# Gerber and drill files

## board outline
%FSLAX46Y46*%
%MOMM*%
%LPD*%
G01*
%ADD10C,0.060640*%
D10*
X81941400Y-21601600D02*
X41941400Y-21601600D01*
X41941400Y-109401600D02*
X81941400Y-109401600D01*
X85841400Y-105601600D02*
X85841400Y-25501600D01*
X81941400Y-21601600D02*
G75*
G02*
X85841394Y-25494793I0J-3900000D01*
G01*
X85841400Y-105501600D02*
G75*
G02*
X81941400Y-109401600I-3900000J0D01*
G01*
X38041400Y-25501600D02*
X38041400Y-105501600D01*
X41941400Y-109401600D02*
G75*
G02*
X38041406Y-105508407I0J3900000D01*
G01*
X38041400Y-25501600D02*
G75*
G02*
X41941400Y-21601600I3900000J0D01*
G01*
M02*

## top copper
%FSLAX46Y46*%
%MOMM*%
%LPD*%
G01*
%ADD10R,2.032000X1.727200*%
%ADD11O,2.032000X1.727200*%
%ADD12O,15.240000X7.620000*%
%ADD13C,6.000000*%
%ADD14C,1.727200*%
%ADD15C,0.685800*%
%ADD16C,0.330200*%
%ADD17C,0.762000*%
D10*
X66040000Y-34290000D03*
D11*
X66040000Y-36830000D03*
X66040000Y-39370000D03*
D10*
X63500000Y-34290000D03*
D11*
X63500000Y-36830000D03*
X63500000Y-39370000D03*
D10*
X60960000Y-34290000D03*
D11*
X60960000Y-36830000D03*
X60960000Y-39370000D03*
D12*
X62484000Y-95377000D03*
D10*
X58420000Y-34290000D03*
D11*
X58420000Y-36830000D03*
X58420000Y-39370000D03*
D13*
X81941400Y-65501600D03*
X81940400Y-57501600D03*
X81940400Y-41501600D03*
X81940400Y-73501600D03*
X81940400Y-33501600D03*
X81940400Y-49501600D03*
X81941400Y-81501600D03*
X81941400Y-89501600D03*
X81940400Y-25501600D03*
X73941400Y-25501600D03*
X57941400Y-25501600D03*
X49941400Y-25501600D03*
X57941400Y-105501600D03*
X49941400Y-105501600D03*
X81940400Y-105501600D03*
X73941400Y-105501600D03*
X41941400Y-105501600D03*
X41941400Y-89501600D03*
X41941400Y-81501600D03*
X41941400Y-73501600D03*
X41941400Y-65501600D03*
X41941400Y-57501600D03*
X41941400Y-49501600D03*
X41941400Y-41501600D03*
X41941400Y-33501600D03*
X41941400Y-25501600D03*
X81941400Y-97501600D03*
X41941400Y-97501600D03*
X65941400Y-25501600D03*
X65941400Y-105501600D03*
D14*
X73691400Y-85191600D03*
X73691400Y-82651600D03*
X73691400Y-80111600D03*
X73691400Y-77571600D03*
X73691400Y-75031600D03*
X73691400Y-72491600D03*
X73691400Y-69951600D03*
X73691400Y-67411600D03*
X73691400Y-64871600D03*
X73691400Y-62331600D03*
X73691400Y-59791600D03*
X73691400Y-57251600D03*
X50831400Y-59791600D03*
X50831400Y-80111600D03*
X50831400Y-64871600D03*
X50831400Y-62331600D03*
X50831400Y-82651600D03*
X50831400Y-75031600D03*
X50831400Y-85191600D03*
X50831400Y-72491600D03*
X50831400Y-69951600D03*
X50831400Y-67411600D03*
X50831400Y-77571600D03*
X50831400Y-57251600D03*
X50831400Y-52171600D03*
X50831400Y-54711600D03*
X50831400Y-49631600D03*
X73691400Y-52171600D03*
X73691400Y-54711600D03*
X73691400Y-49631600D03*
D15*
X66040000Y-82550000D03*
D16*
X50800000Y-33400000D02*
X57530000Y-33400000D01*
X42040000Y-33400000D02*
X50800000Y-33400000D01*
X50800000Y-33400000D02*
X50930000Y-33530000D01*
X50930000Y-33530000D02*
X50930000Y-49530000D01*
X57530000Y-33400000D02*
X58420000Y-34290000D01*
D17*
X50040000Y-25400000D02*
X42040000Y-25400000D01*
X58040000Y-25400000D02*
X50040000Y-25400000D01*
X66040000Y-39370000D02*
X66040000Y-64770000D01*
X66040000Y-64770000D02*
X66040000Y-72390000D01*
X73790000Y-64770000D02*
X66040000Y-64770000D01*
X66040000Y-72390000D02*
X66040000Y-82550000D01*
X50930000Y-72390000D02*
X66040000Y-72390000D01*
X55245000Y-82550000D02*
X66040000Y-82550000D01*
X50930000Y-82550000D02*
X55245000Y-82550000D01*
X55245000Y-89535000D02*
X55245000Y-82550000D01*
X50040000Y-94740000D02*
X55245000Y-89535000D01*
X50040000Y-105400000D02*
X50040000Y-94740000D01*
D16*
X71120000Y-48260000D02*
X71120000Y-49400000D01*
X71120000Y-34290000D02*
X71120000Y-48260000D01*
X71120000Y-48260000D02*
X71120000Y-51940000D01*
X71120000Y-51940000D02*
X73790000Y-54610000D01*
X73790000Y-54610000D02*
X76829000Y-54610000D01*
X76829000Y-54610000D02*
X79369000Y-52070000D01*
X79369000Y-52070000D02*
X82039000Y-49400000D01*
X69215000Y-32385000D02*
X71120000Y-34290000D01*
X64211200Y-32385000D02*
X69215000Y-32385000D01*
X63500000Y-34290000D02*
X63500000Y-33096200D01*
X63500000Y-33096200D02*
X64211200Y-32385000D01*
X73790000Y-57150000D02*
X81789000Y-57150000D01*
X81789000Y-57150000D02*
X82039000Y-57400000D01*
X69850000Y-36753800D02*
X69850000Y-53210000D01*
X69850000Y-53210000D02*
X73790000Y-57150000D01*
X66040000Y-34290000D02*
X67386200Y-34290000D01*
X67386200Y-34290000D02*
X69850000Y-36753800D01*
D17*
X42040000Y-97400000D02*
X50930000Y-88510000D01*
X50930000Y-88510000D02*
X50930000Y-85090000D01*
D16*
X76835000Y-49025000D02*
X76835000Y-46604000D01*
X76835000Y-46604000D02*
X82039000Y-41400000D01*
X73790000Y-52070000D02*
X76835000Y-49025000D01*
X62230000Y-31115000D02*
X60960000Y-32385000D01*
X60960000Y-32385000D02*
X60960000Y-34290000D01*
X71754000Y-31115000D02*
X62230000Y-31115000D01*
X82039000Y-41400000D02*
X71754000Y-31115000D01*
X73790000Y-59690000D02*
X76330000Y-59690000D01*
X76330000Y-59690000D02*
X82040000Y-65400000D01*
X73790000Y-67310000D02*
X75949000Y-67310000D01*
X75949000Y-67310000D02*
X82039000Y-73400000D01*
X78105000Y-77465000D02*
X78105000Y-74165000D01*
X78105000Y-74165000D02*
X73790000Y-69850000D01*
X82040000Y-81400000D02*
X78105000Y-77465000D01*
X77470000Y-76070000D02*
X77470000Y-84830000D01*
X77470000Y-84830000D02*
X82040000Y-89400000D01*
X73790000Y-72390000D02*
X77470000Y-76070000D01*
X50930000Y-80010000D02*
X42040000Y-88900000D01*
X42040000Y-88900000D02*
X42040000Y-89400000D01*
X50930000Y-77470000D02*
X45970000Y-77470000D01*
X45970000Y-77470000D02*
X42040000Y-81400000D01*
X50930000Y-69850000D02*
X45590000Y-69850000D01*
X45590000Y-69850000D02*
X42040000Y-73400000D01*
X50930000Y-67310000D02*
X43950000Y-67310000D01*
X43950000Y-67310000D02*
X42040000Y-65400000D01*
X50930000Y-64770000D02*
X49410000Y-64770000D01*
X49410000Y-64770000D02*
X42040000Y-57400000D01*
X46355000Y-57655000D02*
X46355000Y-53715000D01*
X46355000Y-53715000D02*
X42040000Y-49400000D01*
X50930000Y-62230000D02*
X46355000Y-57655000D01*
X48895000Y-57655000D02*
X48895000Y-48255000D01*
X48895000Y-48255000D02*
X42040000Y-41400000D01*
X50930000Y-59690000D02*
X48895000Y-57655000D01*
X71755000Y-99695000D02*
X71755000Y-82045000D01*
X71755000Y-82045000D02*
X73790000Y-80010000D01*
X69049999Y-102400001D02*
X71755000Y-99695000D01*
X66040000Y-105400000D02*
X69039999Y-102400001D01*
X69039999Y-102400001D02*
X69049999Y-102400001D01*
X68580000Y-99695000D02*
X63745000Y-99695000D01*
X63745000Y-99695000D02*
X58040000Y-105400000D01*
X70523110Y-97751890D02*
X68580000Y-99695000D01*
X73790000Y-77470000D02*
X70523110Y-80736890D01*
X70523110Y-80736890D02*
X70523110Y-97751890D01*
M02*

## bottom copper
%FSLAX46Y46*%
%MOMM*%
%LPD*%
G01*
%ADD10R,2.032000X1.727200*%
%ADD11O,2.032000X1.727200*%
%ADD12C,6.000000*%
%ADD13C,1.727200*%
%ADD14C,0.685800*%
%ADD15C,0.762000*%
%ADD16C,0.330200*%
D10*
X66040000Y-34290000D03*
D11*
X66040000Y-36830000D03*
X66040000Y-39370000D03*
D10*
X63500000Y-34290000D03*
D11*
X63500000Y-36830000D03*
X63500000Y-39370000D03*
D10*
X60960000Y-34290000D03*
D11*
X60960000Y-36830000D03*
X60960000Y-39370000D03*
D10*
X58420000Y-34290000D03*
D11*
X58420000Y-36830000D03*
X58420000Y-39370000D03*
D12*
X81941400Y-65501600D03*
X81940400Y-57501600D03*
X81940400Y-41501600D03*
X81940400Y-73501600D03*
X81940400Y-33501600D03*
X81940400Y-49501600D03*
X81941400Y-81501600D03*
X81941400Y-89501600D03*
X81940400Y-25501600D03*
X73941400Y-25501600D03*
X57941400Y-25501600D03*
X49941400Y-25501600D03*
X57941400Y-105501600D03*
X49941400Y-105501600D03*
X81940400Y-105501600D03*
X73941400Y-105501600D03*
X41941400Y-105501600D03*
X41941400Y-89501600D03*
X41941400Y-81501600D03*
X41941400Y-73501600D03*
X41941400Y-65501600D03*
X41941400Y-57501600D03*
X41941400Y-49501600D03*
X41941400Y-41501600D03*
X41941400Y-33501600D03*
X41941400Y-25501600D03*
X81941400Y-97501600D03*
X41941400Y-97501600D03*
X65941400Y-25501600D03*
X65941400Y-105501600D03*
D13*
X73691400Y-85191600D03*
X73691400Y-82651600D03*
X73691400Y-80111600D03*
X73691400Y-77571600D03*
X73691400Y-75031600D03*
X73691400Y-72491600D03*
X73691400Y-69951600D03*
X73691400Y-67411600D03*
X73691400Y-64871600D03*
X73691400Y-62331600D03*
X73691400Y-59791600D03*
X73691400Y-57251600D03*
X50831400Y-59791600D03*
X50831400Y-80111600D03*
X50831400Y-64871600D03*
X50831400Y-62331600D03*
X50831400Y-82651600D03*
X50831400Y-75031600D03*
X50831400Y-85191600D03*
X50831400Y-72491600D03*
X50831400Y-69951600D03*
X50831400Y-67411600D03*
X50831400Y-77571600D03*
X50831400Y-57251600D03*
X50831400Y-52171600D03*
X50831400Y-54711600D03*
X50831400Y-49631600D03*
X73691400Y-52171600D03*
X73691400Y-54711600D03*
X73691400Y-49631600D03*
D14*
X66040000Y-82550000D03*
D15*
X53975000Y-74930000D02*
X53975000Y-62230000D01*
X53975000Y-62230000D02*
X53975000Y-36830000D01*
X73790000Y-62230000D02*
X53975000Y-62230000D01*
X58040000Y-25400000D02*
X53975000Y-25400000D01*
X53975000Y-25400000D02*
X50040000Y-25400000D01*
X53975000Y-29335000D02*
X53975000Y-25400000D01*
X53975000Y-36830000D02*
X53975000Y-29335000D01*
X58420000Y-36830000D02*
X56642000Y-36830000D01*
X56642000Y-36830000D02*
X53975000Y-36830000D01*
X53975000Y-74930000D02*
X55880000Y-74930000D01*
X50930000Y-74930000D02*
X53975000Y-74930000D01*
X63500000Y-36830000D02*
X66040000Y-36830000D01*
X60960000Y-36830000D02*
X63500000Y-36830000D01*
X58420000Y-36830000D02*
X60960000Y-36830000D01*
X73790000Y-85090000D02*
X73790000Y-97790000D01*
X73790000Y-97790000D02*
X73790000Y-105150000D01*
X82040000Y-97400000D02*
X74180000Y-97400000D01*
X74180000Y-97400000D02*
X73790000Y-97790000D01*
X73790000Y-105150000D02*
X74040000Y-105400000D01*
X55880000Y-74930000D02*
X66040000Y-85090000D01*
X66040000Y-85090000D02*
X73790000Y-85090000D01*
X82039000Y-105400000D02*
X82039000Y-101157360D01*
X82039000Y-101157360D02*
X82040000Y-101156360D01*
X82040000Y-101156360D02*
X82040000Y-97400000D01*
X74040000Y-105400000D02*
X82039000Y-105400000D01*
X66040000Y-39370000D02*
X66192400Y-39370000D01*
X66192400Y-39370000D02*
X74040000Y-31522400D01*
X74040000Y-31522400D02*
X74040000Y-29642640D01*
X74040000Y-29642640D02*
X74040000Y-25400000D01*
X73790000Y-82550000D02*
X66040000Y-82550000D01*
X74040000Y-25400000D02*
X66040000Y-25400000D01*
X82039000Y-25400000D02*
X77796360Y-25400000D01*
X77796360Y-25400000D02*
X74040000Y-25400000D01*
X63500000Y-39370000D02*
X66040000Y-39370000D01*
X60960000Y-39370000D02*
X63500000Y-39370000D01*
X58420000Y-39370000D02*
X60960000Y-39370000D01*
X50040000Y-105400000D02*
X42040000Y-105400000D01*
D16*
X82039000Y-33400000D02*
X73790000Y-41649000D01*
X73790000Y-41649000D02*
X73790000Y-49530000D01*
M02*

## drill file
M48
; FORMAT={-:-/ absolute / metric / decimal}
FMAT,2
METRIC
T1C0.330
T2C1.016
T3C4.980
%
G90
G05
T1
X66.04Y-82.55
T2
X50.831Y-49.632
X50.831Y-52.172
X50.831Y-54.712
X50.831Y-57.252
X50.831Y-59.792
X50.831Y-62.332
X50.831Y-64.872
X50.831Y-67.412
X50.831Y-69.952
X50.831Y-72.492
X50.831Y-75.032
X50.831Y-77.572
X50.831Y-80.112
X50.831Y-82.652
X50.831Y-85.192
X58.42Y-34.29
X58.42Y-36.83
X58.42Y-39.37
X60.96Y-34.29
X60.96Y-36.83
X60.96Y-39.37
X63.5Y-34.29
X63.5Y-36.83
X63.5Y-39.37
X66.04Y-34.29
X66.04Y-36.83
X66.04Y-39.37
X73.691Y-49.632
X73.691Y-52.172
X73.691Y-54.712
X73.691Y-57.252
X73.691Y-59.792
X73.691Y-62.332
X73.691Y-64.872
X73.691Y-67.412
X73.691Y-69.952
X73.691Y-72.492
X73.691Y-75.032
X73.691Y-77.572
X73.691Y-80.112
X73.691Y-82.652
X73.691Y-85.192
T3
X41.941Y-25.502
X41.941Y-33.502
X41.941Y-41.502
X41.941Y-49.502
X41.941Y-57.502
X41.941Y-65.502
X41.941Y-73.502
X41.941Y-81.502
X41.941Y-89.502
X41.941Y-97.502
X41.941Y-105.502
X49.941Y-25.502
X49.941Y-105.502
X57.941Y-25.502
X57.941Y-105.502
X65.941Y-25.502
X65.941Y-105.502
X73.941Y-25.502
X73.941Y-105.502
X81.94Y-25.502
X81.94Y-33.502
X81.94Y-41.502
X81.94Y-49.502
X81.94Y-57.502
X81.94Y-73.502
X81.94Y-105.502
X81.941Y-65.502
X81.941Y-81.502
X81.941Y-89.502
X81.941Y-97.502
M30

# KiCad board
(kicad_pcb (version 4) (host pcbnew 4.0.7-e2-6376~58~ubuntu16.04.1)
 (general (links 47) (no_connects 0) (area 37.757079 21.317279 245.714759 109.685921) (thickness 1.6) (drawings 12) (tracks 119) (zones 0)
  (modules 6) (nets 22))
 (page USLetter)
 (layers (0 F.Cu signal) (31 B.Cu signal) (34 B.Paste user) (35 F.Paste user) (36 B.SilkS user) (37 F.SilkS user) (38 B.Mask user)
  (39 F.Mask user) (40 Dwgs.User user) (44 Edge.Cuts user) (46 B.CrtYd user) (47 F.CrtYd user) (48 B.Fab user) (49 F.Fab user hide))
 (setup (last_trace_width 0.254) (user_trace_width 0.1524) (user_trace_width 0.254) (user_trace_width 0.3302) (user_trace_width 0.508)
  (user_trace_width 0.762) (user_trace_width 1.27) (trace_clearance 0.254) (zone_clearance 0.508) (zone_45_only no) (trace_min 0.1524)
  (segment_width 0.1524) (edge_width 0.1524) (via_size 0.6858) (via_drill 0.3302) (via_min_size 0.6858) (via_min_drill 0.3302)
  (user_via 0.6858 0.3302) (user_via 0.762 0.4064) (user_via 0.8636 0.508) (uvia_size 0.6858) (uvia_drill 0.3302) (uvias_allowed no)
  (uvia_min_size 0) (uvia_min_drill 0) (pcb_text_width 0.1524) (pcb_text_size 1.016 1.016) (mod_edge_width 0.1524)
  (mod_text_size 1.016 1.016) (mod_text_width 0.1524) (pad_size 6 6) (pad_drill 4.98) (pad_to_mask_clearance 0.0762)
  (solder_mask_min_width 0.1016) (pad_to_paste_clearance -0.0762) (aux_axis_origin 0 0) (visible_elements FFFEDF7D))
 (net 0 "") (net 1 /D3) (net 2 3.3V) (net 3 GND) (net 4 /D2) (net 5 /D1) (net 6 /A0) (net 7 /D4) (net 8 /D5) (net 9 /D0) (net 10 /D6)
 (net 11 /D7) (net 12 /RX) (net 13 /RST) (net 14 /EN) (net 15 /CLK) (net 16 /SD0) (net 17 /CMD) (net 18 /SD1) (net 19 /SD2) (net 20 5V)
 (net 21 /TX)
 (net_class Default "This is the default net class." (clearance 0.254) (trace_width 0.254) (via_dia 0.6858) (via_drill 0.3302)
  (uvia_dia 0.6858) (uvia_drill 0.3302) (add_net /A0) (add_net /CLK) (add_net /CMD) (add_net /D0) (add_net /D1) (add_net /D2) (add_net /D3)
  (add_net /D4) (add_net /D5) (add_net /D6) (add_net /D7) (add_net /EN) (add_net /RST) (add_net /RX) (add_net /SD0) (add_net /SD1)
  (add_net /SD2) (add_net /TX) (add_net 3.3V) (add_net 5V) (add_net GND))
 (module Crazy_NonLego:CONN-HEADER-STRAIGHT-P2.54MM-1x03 (layer F.Cu) (at 66.04 34.29)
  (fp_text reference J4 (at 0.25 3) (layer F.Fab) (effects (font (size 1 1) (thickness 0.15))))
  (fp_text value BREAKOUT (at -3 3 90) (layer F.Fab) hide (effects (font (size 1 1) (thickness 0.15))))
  (pad 1 thru_hole rect (at 0 0) (size 2.032 1.7272) (drill 1.016) (layers *.Cu *.Mask F.SilkS) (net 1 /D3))
  (pad 2 thru_hole oval (at 0 2.54) (size 2.032 1.7272) (drill 1.016) (layers *.Cu *.Mask F.SilkS) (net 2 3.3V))
  (pad 3 thru_hole oval (at 0 5.08) (size 2.032 1.7272) (drill 1.016) (layers *.Cu *.Mask F.SilkS) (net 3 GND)))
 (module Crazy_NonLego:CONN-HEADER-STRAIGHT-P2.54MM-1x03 (layer F.Cu) (at 63.5 34.29)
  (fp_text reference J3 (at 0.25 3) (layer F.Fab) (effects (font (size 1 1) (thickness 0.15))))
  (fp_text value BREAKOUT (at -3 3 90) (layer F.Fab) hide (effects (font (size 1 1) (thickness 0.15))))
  (pad 1 thru_hole rect (at 0 0) (size 2.032 1.7272) (drill 1.016) (layers *.Cu *.Mask F.SilkS) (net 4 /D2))
  (pad 2 thru_hole oval (at 0 2.54) (size 2.032 1.7272) (drill 1.016) (layers *.Cu *.Mask F.SilkS) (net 2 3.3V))
  (pad 3 thru_hole oval (at 0 5.08) (size 2.032 1.7272) (drill 1.016) (layers *.Cu *.Mask F.SilkS) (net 3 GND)))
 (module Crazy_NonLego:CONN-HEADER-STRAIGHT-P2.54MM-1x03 (layer F.Cu) (at 60.96 34.29)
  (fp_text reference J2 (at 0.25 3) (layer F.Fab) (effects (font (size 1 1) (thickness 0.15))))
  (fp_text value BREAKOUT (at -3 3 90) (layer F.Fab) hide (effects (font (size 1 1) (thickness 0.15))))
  (pad 1 thru_hole rect (at 0 0) (size 2.032 1.7272) (drill 1.016) (layers *.Cu *.Mask F.SilkS) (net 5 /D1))
  (pad 2 thru_hole oval (at 0 2.54) (size 2.032 1.7272) (drill 1.016) (layers *.Cu *.Mask F.SilkS) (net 2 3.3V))
  (pad 3 thru_hole oval (at 0 5.08) (size 2.032 1.7272) (drill 1.016) (layers *.Cu *.Mask F.SilkS) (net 3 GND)))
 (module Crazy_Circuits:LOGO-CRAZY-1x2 (layer F.Cu) (at 62.484 99.314)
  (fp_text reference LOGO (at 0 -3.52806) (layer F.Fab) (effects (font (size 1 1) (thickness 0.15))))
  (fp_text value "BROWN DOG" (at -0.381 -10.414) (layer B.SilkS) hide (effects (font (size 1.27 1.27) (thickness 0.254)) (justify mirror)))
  (pad BG smd oval (at 0 -3.937) (size 15.24 7.62) (layers F.Cu)))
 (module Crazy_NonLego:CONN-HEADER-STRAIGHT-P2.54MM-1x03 (layer F.Cu) (at 58.42 34.29)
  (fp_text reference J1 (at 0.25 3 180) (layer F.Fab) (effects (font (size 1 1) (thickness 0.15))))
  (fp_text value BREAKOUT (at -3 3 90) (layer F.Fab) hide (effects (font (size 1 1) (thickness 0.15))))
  (pad 1 thru_hole rect (at 0 0) (size 2.032 1.7272) (drill 1.016) (layers *.Cu *.Mask F.SilkS) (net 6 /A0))
  (pad 2 thru_hole oval (at 0 2.54) (size 2.032 1.7272) (drill 1.016) (layers *.Cu *.Mask F.SilkS) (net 2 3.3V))
  (pad 3 thru_hole oval (at 0 5.08) (size 2.032 1.7272) (drill 1.016) (layers *.Cu *.Mask F.SilkS) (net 3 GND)))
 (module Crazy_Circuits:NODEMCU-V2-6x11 (layer F.Cu) (at 41.9414 25.5016)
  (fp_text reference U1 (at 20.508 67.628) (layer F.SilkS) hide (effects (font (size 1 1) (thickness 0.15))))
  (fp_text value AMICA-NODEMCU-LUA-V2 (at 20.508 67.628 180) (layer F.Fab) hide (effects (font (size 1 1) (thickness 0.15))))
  (fp_line (start 40 -3.9) (end 0 -3.9) (layer Edge.Cuts) (width 0.06064))
  (fp_line (start 0 83.9) (end 40 83.9) (layer Edge.Cuts) (width 0.06064))
  (fp_line (start 43.9 80.1) (end 43.9 0) (layer Edge.Cuts) (width 0.06064))
  (fp_arc (start 40 0) (end 40 -3.9) (angle 89.9) (layer Edge.Cuts) (width 0.06064))
  (fp_arc (start 40 80) (end 43.9 80) (angle 90) (layer Edge.Cuts) (width 0.06064))
  (fp_line (start -3.9 0) (end -3.9 80) (layer Edge.Cuts) (width 0.06064))
  (fp_arc (start 0 80) (end 0 83.9) (angle 89.9) (layer Edge.Cuts) (width 0.06064))
  (fp_arc (start 0 0) (end -3.9 0) (angle 90) (layer Edge.Cuts) (width 0.06064))
  (pad D4 thru_hole circle (at 40 40 270) (size 6 6) (drill 4.98) (layers *.Cu *.Mask) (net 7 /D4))
  (pad D3 thru_hole circle (at 39.999 32 270) (size 6 6) (drill 4.98) (layers *.Cu *.Mask) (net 1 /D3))
  (pad D1 thru_hole circle (at 39.999 16 270) (size 6 6) (drill 4.98) (layers *.Cu *.Mask) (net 5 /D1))
  (pad D5 thru_hole circle (at 39.999 48 270) (size 6 6) (drill 4.98) (layers *.Cu *.Mask) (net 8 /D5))
  (pad D0 thru_hole circle (at 39.999 8 270) (size 6 6) (drill 4.98) (layers *.Cu *.Mask) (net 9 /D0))
  (pad D2 thru_hole circle (at 39.999 24 270) (size 6 6) (drill 4.98) (layers *.Cu *.Mask) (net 4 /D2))
  (pad D6 thru_hole circle (at 40 56 270) (size 6 6) (drill 4.98) (layers *.Cu *.Mask) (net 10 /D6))
  (pad D7 thru_hole circle (at 40 64 270) (size 6 6) (drill 4.98) (layers *.Cu *.Mask) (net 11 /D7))
  (pad GND thru_hole circle (at 39.999 0 270) (size 6 6) (drill 4.98) (layers *.Cu *.Mask) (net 3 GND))
  (pad GND thru_hole circle (at 32 0 270) (size 6 6) (drill 4.98) (layers *.Cu *.Mask) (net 3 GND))
  (pad 3V3 thru_hole circle (at 16 0 270) (size 6 6) (drill 4.98) (layers *.Cu *.Mask) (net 2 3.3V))
  (pad 3V3 thru_hole circle (at 8 0 270) (size 6 6) (drill 4.98) (layers *.Cu *.Mask) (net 2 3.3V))
  (pad RX thru_hole circle (at 16 80 270) (size 6 6) (drill 4.98) (layers *.Cu *.Mask) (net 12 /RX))
  (pad GND thru_hole circle (at 8 80 270) (size 6 6) (drill 4.98) (layers *.Cu *.Mask) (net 3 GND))
  (pad 3V3 thru_hole circle (at 39.999 80 270) (size 6 6) (drill 4.98) (layers *.Cu *.Mask) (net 2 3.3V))
  (pad 3V3 thru_hole circle (at 32 80 270) (size 6 6) (drill 4.98) (layers *.Cu *.Mask) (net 2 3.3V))
  (pad GND thru_hole circle (at 0 80 270) (size 6 6) (drill 4.98) (layers *.Cu *.Mask) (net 3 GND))
  (pad RST thru_hole circle (at 0 64 270) (size 6 6) (drill 4.98) (layers *.Cu *.Mask) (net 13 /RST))
  (pad EN thru_hole circle (at 0 56 270) (size 6 6) (drill 4.98) (layers *.Cu *.Mask) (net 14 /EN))
  (pad CLK thru_hole circle (at 0 48 270) (size 6 6) (drill 4.98) (layers *.Cu *.Mask) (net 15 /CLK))
  (pad SD0 thru_hole circle (at 0 40 270) (size 6 6) (drill 4.98) (layers *.Cu *.Mask) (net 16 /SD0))
  (pad CMD thru_hole circle (at 0 32 270) (size 6 6) (drill 4.98) (layers *.Cu *.Mask) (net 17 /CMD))
  (pad SD1 thru_hole circle (at 0 24 270) (size 6 6) (drill 4.98) (layers *.Cu *.Mask) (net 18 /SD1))
  (pad SD2 thru_hole circle (at 0 16 270) (size 6 6) (drill 4.98) (layers *.Cu *.Mask) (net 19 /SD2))
  (pad A0 thru_hole circle (at 0 8 270) (size 6 6) (drill 4.98) (layers *.Cu *.Mask) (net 6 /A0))
  (pad 3V3 thru_hole circle (at 0 0 270) (size 6 6) (drill 4.98) (layers *.Cu *.Mask) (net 2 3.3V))
  (pad 3V3 thru_hole circle (at 40 72 270) (size 6 6) (drill 4.98) (layers *.Cu *.Mask) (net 2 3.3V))
  (pad VIN thru_hole circle (at 0 72 270) (size 6 6) (drill 4.98) (layers *.Cu *.Mask) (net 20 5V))
  (pad GND thru_hole circle (at 24 0 270) (size 6 6) (drill 4.98) (layers *.Cu *.Mask) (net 3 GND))
  (pad TX thru_hole circle (at 24 80 270) (size 6 6) (drill 4.98) (layers *.Cu *.Mask) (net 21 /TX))
  (pad 3V3 thru_hole circle (at 31.75 59.69 180) (size 1.7272 1.7272) (drill 1.016) (layers *.Cu *.Mask F.SilkS) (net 2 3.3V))
  (pad GND thru_hole circle (at 31.75 57.15 180) (size 1.7272 1.7272) (drill 1.016) (layers *.Cu *.Mask F.SilkS) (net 3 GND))
  (pad TX thru_hole circle (at 31.75 54.61 180) (size 1.7272 1.7272) (drill 1.016) (layers *.Cu *.Mask F.SilkS) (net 21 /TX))
  (pad RX thru_hole circle (at 31.75 52.07 180) (size 1.7272 1.7272) (drill 1.016) (layers *.Cu *.Mask F.SilkS) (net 12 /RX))
  (pad D8 thru_hole circle (at 31.75 49.53 180) (size 1.7272 1.7272) (drill 1.016) (layers *.Cu *.Mask F.SilkS))
  (pad D7 thru_hole circle (at 31.75 46.99 180) (size 1.7272 1.7272) (drill 1.016) (layers *.Cu *.Mask F.SilkS) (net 11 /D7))
  (pad D6 thru_hole circle (at 31.75 44.45 180) (size 1.7272 1.7272) (drill 1.016) (layers *.Cu *.Mask F.SilkS) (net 10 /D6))
  (pad D5 thru_hole circle (at 31.75 41.91 180) (size 1.7272 1.7272) (drill 1.016) (layers *.Cu *.Mask F.SilkS) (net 8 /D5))
  (pad GND thru_hole circle (at 31.75 39.37 180) (size 1.7272 1.7272) (drill 1.016) (layers *.Cu *.Mask F.SilkS) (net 3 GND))
  (pad 3V3 thru_hole circle (at 31.75 36.83 180) (size 1.7272 1.7272) (drill 1.016) (layers *.Cu *.Mask F.SilkS) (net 2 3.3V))
  (pad D4 thru_hole circle (at 31.75 34.29 180) (size 1.7272 1.7272) (drill 1.016) (layers *.Cu *.Mask F.SilkS) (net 7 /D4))
  (pad D3 thru_hole circle (at 31.75 31.75 180) (size 1.7272 1.7272) (drill 1.016) (layers *.Cu *.Mask F.SilkS) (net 1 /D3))
  (pad SD2 thru_hole circle (at 8.89 34.29 180) (size 1.7272 1.7272) (drill 1.016) (layers *.Cu *.Mask F.SilkS) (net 19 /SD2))
  (pad RST thru_hole circle (at 8.89 54.61 180) (size 1.7272 1.7272) (drill 1.016) (layers *.Cu *.Mask F.SilkS) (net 13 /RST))
  (pad CMD thru_hole circle (at 8.89 39.37 180) (size 1.7272 1.7272) (drill 1.016) (layers *.Cu *.Mask F.SilkS) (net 17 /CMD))
  (pad SD1 thru_hole circle (at 8.89 36.83 180) (size 1.7272 1.7272) (drill 1.016) (layers *.Cu *.Mask F.SilkS) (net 18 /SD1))
  (pad GND thru_hole circle (at 8.89 57.15 180) (size 1.7272 1.7272) (drill 1.016) (layers *.Cu *.Mask F.SilkS) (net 3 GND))
  (pad 3V3 thru_hole circle (at 8.89 49.53 180) (size 1.7272 1.7272) (drill 1.016) (layers *.Cu *.Mask F.SilkS) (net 2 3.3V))
  (pad VIN thru_hole circle (at 8.89 59.69 180) (size 1.7272 1.7272) (drill 1.016) (layers *.Cu *.Mask F.SilkS) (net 20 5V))
  (pad GND thru_hole circle (at 8.89 46.99 180) (size 1.7272 1.7272) (drill 1.016) (layers *.Cu *.Mask F.SilkS) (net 3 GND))
  (pad CLK thru_hole circle (at 8.89 44.45 180) (size 1.7272 1.7272) (drill 1.016) (layers *.Cu *.Mask F.SilkS) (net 15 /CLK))
  (pad SD0 thru_hole circle (at 8.89 41.91 180) (size 1.7272 1.7272) (drill 1.016) (layers *.Cu *.Mask F.SilkS) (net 16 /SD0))
  (pad EN thru_hole circle (at 8.89 52.07 180) (size 1.7272 1.7272) (drill 1.016) (layers *.Cu *.Mask F.SilkS) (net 14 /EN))
  (pad SD3 thru_hole circle (at 8.89 31.75 180) (size 1.7272 1.7272) (drill 1.016) (layers *.Cu *.Mask F.SilkS))
  (pad RSV thru_hole circle (at 8.89 26.67 180) (size 1.7272 1.7272) (drill 1.016) (layers *.Cu *.Mask F.SilkS))
  (pad RSV thru_hole circle (at 8.89 29.21 180) (size 1.7272 1.7272) (drill 1.016) (layers *.Cu *.Mask F.SilkS))
  (pad A0 thru_hole circle (at 8.89 24.13 180) (size 1.7272 1.7272) (drill 1.016) (layers *.Cu *.Mask F.SilkS) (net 6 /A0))
  (pad D1 thru_hole circle (at 31.75 26.67 180) (size 1.7272 1.7272) (drill 1.016) (layers *.Cu *.Mask F.SilkS) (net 5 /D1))
  (pad D2 thru_hole circle (at 31.75 29.21 180) (size 1.7272 1.7272) (drill 1.016) (layers *.Cu *.Mask F.SilkS) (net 4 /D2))
  (pad D0 thru_hole circle (at 31.75 24.13 180) (size 1.7272 1.7272) (drill 1.016) (layers *.Cu *.Mask F.SilkS) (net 9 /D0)))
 (segment (start 50.8 33.4) (end 57.53 33.4) (width 0.3302) (layer F.Cu) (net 6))
 (segment (start 42.04 33.4) (end 50.8 33.4) (width 0.3302) (layer F.Cu) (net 6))
 (segment (start 50.8 33.4) (end 50.93 33.53) (width 0.3302) (layer F.Cu) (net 6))
 (segment (start 50.93 33.53) (end 50.93 49.53) (width 0.3302) (layer F.Cu) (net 6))
 (segment (start 57.53 33.4) (end 58.42 34.29) (width 0.3302) (layer F.Cu) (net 6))
 (segment (start 53.975 74.93) (end 53.975 62.23) (width 0.762) (layer B.Cu) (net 2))
 (segment (start 53.975 62.23) (end 53.975 36.83) (width 0.762) (layer B.Cu) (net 2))
 (segment (start 73.79 62.23) (end 53.975 62.23) (width 0.762) (layer B.Cu) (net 2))
 (segment (start 50.04 25.4) (end 42.04 25.4) (width 0.762) (layer F.Cu) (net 2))
 (segment (start 58.04 25.4) (end 50.04 25.4) (width 0.762) (layer F.Cu) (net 2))
 (segment (start 58.04 25.4) (end 53.975 25.4) (width 0.762) (layer B.Cu) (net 2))
 (segment (start 53.975 25.4) (end 50.04 25.4) (width 0.762) (layer B.Cu) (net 2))
 (segment (start 53.975 29.335) (end 53.975 25.4) (width 0.762) (layer B.Cu) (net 2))
 (segment (start 53.975 36.83) (end 53.975 29.335) (width 0.762) (layer B.Cu) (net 2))
 (segment (start 58.42 36.83) (end 56.642 36.83) (width 0.762) (layer B.Cu) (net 2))
 (segment (start 56.642 36.83) (end 53.975 36.83) (width 0.762) (layer B.Cu) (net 2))
 (segment (start 53.975 74.93) (end 55.88 74.93) (width 0.762) (layer B.Cu) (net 2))
 (segment (start 50.93 74.93) (end 53.975 74.93) (width 0.762) (layer B.Cu) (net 2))
 (segment (start 63.5 36.83) (end 66.04 36.83) (width 0.762) (layer B.Cu) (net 2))
 (segment (start 60.96 36.83) (end 63.5 36.83) (width 0.762) (layer B.Cu) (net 2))
 (segment (start 58.42 36.83) (end 60.96 36.83) (width 0.762) (layer B.Cu) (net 2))
 (segment (start 73.79 85.09) (end 73.79 97.79) (width 0.762) (layer B.Cu) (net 2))
 (segment (start 73.79 97.79) (end 73.79 105.15) (width 0.762) (layer B.Cu) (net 2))
 (segment (start 82.04 97.4) (end 74.18 97.4) (width 0.762) (layer B.Cu) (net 2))
 (segment (start 74.18 97.4) (end 73.79 97.79) (width 0.762) (layer B.Cu) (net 2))
 (segment (start 73.79 105.15) (end 74.04 105.4) (width 0.762) (layer B.Cu) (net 2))
 (segment (start 55.88 74.93) (end 66.04 85.09) (width 0.762) (layer B.Cu) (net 2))
 (segment (start 66.04 85.09) (end 73.79 85.09) (width 0.762) (layer B.Cu) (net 2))
 (segment (start 82.039 105.4) (end 82.039 101.15736) (width 0.762) (layer B.Cu) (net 2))
 (segment (start 82.039 101.15736) (end 82.04 101.15636) (width 0.762) (layer B.Cu) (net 2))
 (segment (start 82.04 101.15636) (end 82.04 97.4) (width 0.762) (layer B.Cu) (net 2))
 (segment (start 74.04 105.4) (end 82.039 105.4) (width 0.762) (layer B.Cu) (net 2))
 (segment (start 66.04 39.37) (end 66.1924 39.37) (width 0.762) (layer B.Cu) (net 3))
 (segment (start 66.1924 39.37) (end 74.04 31.5224) (width 0.762) (layer B.Cu) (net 3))
 (segment (start 74.04 31.5224) (end 74.04 29.64264) (width 0.762) (layer B.Cu) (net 3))
 (segment (start 74.04 29.64264) (end 74.04 25.4) (width 0.762) (layer B.Cu) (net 3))
 (segment (start 73.79 82.55) (end 66.04 82.55) (width 0.762) (layer B.Cu) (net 3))
 (via (at 66.04 82.55) (size 0.6858) (drill 0.3302) (layers F.Cu B.Cu) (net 3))
 (segment (start 66.04 39.37) (end 66.04 64.77) (width 0.762) (layer F.Cu) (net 3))
 (segment (start 66.04 64.77) (end 66.04 72.39) (width 0.762) (layer F.Cu) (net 3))
 (segment (start 73.79 64.77) (end 66.04 64.77) (width 0.762) (layer F.Cu) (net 3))
 (segment (start 66.04 72.39) (end 66.04 82.55) (width 0.762) (layer F.Cu) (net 3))
 (segment (start 50.93 72.39) (end 66.04 72.39) (width 0.762) (layer F.Cu) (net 3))
 (segment (start 55.245 82.55) (end 66.04 82.55) (width 0.762) (layer F.Cu) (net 3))
 (segment (start 74.04 25.4) (end 66.04 25.4) (width 0.762) (layer B.Cu) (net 3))
 (segment (start 82.039 25.4) (end 77.79636 25.4) (width 0.762) (layer B.Cu) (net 3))
 (segment (start 77.79636 25.4) (end 74.04 25.4) (width 0.762) (layer B.Cu) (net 3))
 (segment (start 63.5 39.37) (end 66.04 39.37) (width 0.762) (layer B.Cu) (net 3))
 (segment (start 60.96 39.37) (end 63.5 39.37) (width 0.762) (layer B.Cu) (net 3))
 (segment (start 58.42 39.37) (end 60.96 39.37) (width 0.762) (layer B.Cu) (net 3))
 (segment (start 50.04 105.4) (end 42.04 105.4) (width 0.762) (layer B.Cu) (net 3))
 (segment (start 50.93 82.55) (end 55.245 82.55) (width 0.762) (layer F.Cu) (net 3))
 (segment (start 55.245 89.535) (end 55.245 82.55) (width 0.762) (layer F.Cu) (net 3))
 (segment (start 50.04 94.74) (end 55.245 89.535) (width 0.762) (layer F.Cu) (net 3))
 (segment (start 50.04 105.4) (end 50.04 94.74) (width 0.762) (layer F.Cu) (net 3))
 (segment (start 71.12 48.26) (end 71.12 49.4) (width 0.3302) (layer F.Cu) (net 4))
 (segment (start 71.12 34.29) (end 71.12 48.26) (width 0.3302) (layer F.Cu) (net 4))
 (segment (start 71.12 48.26) (end 71.12 51.94) (width 0.3302) (layer F.Cu) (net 4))
 (segment (start 71.12 51.94) (end 73.79 54.61) (width 0.3302) (layer F.Cu) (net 4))
 (segment (start 73.79 54.61) (end 76.829 54.61) (width 0.3302) (layer F.Cu) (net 4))
 (segment (start 76.829 54.61) (end 79.369 52.07) (width 0.3302) (layer F.Cu) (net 4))
 (segment (start 79.369 52.07) (end 82.039 49.4) (width 0.3302) (layer F.Cu) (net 4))
 (segment (start 69.215 32.385) (end 71.12 34.29) (width 0.3302) (layer F.Cu) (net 4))
 (segment (start 64.2112 32.385) (end 69.215 32.385) (width 0.3302) (layer F.Cu) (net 4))
 (segment (start 63.5 34.29) (end 63.5 33.0962) (width 0.3302) (layer F.Cu) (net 4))
 (segment (start 63.5 33.0962) (end 64.2112 32.385) (width 0.3302) (layer F.Cu) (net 4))
 (segment (start 73.79 57.15) (end 81.789 57.15) (width 0.3302) (layer F.Cu) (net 1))
 (segment (start 81.789 57.15) (end 82.039 57.4) (width 0.3302) (layer F.Cu) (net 1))
 (segment (start 69.85 36.7538) (end 69.85 53.21) (width 0.3302) (layer F.Cu) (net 1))
 (segment (start 69.85 53.21) (end 73.79 57.15) (width 0.3302) (layer F.Cu) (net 1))
 (segment (start 66.04 34.29) (end 67.3862 34.29) (width 0.3302) (layer F.Cu) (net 1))
 (segment (start 67.3862 34.29) (end 69.85 36.7538) (width 0.3302) (layer F.Cu) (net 1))
 (segment (start 42.04 97.4) (end 50.93 88.51) (width 0.762) (layer F.Cu) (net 20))
 (segment (start 50.93 88.51) (end 50.93 85.09) (width 0.762) (layer F.Cu) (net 20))
 (segment (start 76.835 49.025) (end 76.835 46.604) (width 0.3302) (layer F.Cu) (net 5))
 (segment (start 76.835 46.604) (end 82.039 41.4) (width 0.3302) (layer F.Cu) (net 5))
 (segment (start 73.79 52.07) (end 76.835 49.025) (width 0.3302) (layer F.Cu) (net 5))
 (segment (start 62.23 31.115) (end 60.96 32.385) (width 0.3302) (layer F.Cu) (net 5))
 (segment (start 60.96 32.385) (end 60.96 34.29) (width 0.3302) (layer F.Cu) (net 5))
 (segment (start 71.754 31.115) (end 62.23 31.115) (width 0.3302) (layer F.Cu) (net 5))
 (segment (start 82.039 41.4) (end 71.754 31.115) (width 0.3302) (layer F.Cu) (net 5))
 (segment (start 73.79 59.69) (end 76.33 59.69) (width 0.3302) (layer F.Cu) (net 7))
 (segment (start 76.33 59.69) (end 82.04 65.4) (width 0.3302) (layer F.Cu) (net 7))
 (segment (start 73.79 67.31) (end 75.949 67.31) (width 0.3302) (layer F.Cu) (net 8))
 (segment (start 75.949 67.31) (end 82.039 73.4) (width 0.3302) (layer F.Cu) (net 8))
 (segment (start 82.039 33.4) (end 73.79 41.649) (width 0.3302) (layer B.Cu) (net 9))
 (segment (start 73.79 41.649) (end 73.79 49.53) (width 0.3302) (layer B.Cu) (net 9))
 (segment (start 78.105 77.465) (end 78.105 74.165) (width 0.3302) (layer F.Cu) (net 10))
 (segment (start 78.105 74.165) (end 73.79 69.85) (width 0.3302) (layer F.Cu) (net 10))
 (segment (start 82.04 81.4) (end 78.105 77.465) (width 0.3302) (layer F.Cu) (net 10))
 (segment (start 77.47 76.07) (end 77.47 84.83) (width 0.3302) (layer F.Cu) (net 11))
 (segment (start 77.47 84.83) (end 82.04 89.4) (width 0.3302) (layer F.Cu) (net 11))
 (segment (start 73.79 72.39) (end 77.47 76.07) (width 0.3302) (layer F.Cu) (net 11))
 (segment (start 50.93 80.01) (end 42.04 88.9) (width 0.3302) (layer F.Cu) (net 13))
 (segment (start 42.04 88.9) (end 42.04 89.4) (width 0.3302) (layer F.Cu) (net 13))
 (segment (start 50.93 77.47) (end 45.97 77.47) (width 0.3302) (layer F.Cu) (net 14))
 (segment (start 45.97 77.47) (end 42.04 81.4) (width 0.3302) (layer F.Cu) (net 14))
 (segment (start 50.93 69.85) (end 45.59 69.85) (width 0.3302) (layer F.Cu) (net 15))
 (segment (start 45.59 69.85) (end 42.04 73.4) (width 0.3302) (layer F.Cu) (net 15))
 (segment (start 50.93 67.31) (end 43.95 67.31) (width 0.3302) (layer F.Cu) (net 16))
 (segment (start 43.95 67.31) (end 42.04 65.4) (width 0.3302) (layer F.Cu) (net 16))
 (segment (start 50.93 64.77) (end 49.41 64.77) (width 0.3302) (layer F.Cu) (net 17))
 (segment (start 49.41 64.77) (end 42.04 57.4) (width 0.3302) (layer F.Cu) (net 17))
 (segment (start 46.355 57.655) (end 46.355 53.715) (width 0.3302) (layer F.Cu) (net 18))
 (segment (start 46.355 53.715) (end 42.04 49.4) (width 0.3302) (layer F.Cu) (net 18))
 (segment (start 50.93 62.23) (end 46.355 57.655) (width 0.3302) (layer F.Cu) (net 18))
 (segment (start 48.895 57.655) (end 48.895 48.255) (width 0.3302) (layer F.Cu) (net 19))
 (segment (start 48.895 48.255) (end 42.04 41.4) (width 0.3302) (layer F.Cu) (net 19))
 (segment (start 50.93 59.69) (end 48.895 57.655) (width 0.3302) (layer F.Cu) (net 19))
 (segment (start 71.755 99.695) (end 71.755 82.045) (width 0.3302) (layer F.Cu) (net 21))
 (segment (start 71.755 82.045) (end 73.79 80.01) (width 0.3302) (layer F.Cu) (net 21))
 (segment (start 69.049999 102.400001) (end 71.755 99.695) (width 0.3302) (layer F.Cu) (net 21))
 (segment (start 66.04 105.4) (end 69.039999 102.400001) (width 0.3302) (layer F.Cu) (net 21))
 (segment (start 69.039999 102.400001) (end 69.049999 102.400001) (width 0.3302) (layer F.Cu) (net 21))
 (segment (start 68.58 99.695) (end 63.745 99.695) (width 0.3302) (layer F.Cu) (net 12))
 (segment (start 63.745 99.695) (end 58.04 105.4) (width 0.3302) (layer F.Cu) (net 12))
 (segment (start 70.52311 97.75189) (end 68.58 99.695) (width 0.3302) (layer F.Cu) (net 12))
 (segment (start 73.79 77.47) (end 70.52311 80.73689) (width 0.3302) (layer F.Cu) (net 12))
 (segment (start 70.52311 80.73689) (end 70.52311 97.75189) (width 0.3302) (layer F.Cu) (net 12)))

